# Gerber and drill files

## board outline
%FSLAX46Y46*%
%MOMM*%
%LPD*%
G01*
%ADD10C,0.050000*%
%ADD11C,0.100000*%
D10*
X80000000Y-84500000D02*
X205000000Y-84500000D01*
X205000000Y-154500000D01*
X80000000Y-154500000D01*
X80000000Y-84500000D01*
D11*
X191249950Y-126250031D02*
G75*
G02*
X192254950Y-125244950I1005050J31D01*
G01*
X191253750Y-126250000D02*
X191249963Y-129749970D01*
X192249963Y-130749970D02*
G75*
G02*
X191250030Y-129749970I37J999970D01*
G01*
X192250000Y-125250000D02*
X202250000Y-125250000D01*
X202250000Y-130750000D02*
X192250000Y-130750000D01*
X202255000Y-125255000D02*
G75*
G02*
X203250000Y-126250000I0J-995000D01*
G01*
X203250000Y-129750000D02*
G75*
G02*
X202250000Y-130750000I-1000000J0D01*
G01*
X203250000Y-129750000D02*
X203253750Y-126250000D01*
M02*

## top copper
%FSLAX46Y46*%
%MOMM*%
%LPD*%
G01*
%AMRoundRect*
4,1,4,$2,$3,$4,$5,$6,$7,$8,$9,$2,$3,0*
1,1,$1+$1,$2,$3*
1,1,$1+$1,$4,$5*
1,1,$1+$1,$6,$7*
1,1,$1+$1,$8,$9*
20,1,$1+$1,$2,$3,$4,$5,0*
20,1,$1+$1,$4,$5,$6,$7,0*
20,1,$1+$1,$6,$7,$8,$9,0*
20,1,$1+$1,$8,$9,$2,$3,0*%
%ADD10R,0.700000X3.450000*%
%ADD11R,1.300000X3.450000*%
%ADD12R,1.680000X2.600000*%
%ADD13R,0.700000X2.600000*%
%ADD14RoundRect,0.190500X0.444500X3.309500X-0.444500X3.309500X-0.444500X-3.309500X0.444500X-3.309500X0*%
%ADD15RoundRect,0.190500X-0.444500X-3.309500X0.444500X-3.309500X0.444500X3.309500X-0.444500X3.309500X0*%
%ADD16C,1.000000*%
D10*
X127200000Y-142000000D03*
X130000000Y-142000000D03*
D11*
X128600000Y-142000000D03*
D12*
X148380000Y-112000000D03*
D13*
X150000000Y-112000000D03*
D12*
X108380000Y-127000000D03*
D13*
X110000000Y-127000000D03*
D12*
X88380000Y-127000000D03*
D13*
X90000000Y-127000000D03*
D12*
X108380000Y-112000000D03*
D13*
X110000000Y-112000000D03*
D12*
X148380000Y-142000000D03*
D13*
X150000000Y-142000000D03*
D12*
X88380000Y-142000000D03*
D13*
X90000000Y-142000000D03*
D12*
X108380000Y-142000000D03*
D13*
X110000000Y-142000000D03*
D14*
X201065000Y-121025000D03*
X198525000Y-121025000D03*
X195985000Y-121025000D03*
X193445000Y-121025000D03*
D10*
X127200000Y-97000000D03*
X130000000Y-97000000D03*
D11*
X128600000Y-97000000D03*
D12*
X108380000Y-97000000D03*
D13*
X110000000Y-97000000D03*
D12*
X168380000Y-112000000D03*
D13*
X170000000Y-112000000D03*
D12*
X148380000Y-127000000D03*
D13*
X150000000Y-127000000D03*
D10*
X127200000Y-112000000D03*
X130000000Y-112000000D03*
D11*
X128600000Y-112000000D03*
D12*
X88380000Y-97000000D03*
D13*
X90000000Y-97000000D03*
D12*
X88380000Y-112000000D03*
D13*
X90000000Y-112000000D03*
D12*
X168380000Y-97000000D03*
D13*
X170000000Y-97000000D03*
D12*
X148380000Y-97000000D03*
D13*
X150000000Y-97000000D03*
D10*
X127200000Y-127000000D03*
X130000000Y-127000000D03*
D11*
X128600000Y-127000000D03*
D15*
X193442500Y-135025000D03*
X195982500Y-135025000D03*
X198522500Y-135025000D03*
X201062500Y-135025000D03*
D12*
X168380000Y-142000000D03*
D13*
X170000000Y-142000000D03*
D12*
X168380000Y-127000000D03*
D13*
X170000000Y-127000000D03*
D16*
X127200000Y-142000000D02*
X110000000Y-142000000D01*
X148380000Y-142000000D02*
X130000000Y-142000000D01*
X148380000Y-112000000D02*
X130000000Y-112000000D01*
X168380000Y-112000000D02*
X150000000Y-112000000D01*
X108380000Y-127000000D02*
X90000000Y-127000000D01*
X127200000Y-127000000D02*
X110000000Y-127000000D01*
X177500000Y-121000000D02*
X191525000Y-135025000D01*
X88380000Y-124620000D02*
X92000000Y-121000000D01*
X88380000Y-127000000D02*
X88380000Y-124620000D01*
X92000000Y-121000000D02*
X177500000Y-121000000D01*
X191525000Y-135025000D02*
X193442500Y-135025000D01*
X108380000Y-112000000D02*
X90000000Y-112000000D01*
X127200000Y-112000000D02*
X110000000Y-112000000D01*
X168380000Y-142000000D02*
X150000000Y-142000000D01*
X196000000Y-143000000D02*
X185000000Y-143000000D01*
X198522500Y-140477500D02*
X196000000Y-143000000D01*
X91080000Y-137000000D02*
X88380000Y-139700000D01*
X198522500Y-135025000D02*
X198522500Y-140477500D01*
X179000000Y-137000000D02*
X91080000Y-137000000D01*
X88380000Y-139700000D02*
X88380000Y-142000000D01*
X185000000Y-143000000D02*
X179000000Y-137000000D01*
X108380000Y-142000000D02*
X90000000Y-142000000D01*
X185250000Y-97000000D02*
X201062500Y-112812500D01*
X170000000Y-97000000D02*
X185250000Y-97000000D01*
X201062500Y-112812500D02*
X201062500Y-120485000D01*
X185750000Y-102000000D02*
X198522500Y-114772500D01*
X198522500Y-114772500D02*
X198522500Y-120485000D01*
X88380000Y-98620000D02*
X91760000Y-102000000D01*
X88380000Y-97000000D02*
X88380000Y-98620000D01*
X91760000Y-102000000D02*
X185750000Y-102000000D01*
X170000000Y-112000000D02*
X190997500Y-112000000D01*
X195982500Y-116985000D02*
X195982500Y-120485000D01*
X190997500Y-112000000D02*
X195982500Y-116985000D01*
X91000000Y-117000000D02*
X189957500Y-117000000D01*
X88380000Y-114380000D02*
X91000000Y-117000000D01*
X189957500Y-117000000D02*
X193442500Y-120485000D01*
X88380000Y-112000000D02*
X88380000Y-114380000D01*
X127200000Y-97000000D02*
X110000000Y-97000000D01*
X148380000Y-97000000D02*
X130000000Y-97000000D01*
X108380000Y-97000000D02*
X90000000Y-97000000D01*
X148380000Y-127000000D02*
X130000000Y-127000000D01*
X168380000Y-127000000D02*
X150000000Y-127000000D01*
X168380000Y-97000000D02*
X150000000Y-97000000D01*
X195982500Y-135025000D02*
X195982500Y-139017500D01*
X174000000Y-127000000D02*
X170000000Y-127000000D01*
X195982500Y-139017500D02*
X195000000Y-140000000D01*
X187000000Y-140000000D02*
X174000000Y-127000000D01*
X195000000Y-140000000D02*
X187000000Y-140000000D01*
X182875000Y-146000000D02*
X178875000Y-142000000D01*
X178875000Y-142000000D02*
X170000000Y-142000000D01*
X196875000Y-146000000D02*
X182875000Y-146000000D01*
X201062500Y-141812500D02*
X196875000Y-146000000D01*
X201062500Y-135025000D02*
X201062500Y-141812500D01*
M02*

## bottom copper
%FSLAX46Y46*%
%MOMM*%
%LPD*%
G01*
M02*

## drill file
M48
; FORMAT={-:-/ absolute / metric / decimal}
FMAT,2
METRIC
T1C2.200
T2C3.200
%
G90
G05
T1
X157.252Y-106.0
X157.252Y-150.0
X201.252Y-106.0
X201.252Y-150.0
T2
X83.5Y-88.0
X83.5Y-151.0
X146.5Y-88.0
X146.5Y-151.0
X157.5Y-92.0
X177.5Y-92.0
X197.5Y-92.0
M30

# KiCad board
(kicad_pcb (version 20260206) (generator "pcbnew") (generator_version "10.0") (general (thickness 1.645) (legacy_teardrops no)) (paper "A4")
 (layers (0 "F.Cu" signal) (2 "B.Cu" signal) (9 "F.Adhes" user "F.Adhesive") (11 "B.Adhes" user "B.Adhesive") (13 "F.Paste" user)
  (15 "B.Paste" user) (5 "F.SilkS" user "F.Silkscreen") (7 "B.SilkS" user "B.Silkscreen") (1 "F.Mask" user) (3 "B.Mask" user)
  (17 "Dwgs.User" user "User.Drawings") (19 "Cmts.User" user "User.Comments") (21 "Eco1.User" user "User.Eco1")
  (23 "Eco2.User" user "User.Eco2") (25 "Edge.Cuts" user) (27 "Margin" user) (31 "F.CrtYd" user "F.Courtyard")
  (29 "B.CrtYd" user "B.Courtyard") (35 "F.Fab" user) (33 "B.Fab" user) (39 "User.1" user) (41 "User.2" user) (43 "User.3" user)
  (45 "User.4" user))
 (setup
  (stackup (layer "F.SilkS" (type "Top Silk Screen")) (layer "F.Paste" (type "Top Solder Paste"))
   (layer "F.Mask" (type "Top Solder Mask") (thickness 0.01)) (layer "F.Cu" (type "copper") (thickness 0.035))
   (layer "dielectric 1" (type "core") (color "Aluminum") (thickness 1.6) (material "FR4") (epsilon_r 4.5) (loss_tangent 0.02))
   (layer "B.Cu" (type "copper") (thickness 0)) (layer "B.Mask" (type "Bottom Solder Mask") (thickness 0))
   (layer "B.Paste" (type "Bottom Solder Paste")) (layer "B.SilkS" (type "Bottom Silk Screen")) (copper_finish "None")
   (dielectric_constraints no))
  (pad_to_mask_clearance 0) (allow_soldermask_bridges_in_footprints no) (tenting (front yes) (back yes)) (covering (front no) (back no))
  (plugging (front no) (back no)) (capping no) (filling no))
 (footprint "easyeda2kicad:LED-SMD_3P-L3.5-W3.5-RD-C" (layer "F.Cu") (at 128.6 142)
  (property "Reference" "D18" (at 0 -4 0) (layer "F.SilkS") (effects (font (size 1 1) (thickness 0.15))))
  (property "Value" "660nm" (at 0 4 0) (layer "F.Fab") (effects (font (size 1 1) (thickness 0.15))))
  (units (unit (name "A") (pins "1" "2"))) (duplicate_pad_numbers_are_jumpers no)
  (pad "1" smd rect (at -1.4 0 180) (size 0.7 3.45) (layers "F.Cu" "F.Mask" "F.Paste") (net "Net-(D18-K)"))
  (pad "2" smd rect (at 1.4 0 180) (size 0.7 3.45) (layers "F.Cu" "F.Mask" "F.Paste") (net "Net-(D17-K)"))
  (pad "3" smd rect (at 0 0) (size 1.3 3.45) (layers "F.Cu" "F.Mask" "F.Paste")))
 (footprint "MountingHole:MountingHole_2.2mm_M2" (layer "F.Cu") (at 157.2525 106)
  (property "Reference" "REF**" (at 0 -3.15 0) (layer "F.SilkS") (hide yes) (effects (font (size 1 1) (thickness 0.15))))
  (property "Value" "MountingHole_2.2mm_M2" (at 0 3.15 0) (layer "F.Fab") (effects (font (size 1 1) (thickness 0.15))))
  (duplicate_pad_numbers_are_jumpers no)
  (pad "" np_thru_hole circle (at 0 0) (size 2.2 2.2) (drill 2.2) (layers "*.Cu" "*.Mask")))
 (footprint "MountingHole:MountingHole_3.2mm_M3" (layer "F.Cu") (at 83.5 88)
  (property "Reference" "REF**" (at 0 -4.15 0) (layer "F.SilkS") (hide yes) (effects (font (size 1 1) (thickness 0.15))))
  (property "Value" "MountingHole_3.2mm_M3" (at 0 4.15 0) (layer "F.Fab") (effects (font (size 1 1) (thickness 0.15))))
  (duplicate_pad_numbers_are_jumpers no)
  (pad "" np_thru_hole circle (at 0 0) (size 3.2 3.2) (drill 3.2) (layers "*.Cu" "*.Mask")))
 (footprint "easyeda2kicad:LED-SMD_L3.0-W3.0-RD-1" (layer "F.Cu") (at 149.19 112)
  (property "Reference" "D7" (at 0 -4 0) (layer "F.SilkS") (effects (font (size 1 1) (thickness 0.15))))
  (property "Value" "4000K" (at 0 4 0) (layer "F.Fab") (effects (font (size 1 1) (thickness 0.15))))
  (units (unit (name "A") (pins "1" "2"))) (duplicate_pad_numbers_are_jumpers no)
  (pad "1" smd rect (at -0.81 0 180) (size 1.68 2.6) (layers "F.Cu" "F.Mask" "F.Paste") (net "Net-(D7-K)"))
  (pad "2" smd rect (at 0.81 0 180) (size 0.7 2.6) (layers "F.Cu" "F.Mask" "F.Paste") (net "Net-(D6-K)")))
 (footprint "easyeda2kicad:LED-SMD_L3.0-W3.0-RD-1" (layer "F.Cu") (at 109.19 127)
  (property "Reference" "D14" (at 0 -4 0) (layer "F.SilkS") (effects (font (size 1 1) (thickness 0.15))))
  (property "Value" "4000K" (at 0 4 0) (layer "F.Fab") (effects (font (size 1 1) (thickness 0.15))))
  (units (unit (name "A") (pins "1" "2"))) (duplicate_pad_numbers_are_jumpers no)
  (pad "1" smd rect (at -0.81 0 180) (size 1.68 2.6) (layers "F.Cu" "F.Mask" "F.Paste") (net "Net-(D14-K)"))
  (pad "2" smd rect (at 0.81 0 180) (size 0.7 2.6) (layers "F.Cu" "F.Mask" "F.Paste") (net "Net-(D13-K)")))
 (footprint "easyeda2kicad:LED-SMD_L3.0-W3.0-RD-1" (layer "F.Cu") (at 89.19 127)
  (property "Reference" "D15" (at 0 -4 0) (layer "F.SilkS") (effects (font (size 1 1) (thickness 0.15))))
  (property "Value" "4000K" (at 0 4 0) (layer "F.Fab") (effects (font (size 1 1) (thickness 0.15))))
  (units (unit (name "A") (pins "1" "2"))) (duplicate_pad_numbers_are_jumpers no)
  (pad "1" smd rect (at -0.81 0 180) (size 1.68 2.6) (layers "F.Cu" "F.Mask" "F.Paste") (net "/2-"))
  (pad "2" smd rect (at 0.81 0 180) (size 0.7 2.6) (layers "F.Cu" "F.Mask" "F.Paste") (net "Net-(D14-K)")))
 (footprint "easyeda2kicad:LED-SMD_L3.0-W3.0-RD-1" (layer "F.Cu") (at 109.19 112)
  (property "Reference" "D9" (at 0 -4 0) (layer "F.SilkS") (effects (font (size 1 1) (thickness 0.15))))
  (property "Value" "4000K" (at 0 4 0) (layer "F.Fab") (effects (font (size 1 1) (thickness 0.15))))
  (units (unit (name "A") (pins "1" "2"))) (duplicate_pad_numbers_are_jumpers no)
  (pad "1" smd rect (at -0.81 0 180) (size 1.68 2.6) (layers "F.Cu" "F.Mask" "F.Paste") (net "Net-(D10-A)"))
  (pad "2" smd rect (at 0.81 0 180) (size 0.7 2.6) (layers "F.Cu" "F.Mask" "F.Paste") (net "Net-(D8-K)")))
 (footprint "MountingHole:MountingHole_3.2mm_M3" (layer "F.Cu") (at 83.5 151)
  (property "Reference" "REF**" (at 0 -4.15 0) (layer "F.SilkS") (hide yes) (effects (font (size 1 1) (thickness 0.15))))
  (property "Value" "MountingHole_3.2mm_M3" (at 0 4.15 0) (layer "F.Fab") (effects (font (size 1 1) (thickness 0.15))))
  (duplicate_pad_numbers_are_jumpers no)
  (pad "" np_thru_hole circle (at 0 0) (size 3.2 3.2) (drill 3.2) (layers "*.Cu" "*.Mask")))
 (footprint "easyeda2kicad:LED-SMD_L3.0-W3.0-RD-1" (layer "F.Cu") (at 149.19 142)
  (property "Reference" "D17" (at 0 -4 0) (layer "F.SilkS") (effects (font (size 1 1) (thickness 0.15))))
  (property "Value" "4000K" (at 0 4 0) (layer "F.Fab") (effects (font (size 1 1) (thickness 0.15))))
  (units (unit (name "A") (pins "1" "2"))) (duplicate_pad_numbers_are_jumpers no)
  (pad "1" smd rect (at -0.81 0 180) (size 1.68 2.6) (layers "F.Cu" "F.Mask" "F.Paste") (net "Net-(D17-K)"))
  (pad "2" smd rect (at 0.81 0 180) (size 0.7 2.6) (layers "F.Cu" "F.Mask" "F.Paste") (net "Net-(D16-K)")))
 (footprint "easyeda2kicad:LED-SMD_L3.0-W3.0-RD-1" (layer "F.Cu") (at 89.19 142)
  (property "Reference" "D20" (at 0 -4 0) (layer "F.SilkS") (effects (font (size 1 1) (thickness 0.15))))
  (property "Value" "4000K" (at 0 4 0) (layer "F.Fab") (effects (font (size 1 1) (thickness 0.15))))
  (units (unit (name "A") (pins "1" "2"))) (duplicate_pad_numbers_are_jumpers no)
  (pad "1" smd rect (at -0.81 0 180) (size 1.68 2.6) (layers "F.Cu" "F.Mask" "F.Paste") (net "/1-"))
  (pad "2" smd rect (at 0.81 0 180) (size 0.7 2.6) (layers "F.Cu" "F.Mask" "F.Paste") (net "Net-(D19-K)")))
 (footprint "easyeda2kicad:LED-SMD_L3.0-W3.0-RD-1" (layer "F.Cu") (at 109.19 142)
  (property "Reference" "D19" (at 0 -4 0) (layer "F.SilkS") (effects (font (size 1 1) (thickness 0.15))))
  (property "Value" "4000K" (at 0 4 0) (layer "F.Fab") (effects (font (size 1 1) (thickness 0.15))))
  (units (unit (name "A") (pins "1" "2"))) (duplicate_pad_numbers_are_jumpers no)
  (pad "1" smd rect (at -0.81 0 180) (size 1.68 2.6) (layers "F.Cu" "F.Mask" "F.Paste") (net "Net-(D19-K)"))
  (pad "2" smd rect (at 0.81 0 180) (size 0.7 2.6) (layers "F.Cu" "F.Mask" "F.Paste") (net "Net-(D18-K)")))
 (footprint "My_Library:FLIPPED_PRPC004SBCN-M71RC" (layer "F.Cu") (at 197.255 121.295 180)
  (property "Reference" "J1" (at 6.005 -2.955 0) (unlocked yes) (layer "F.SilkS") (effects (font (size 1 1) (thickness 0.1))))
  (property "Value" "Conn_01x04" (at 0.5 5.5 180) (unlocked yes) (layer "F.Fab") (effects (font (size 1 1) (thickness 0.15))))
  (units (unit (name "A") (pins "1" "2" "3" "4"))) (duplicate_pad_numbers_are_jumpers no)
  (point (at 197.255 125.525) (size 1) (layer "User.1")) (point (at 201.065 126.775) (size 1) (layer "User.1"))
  (pad "1" smd roundrect (at -3.81 0.27 180) (size 1.27 7) (layers "F.Cu" "F.Mask" "F.Paste") (roundrect_rratio 0.15) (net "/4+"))
  (pad "2" smd roundrect (at -1.27 0.27 180) (size 1.27 7) (layers "F.Cu" "F.Mask" "F.Paste") (roundrect_rratio 0.15) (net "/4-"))
  (pad "3" smd roundrect (at 1.27 0.27 180) (size 1.27 7) (layers "F.Cu" "F.Mask" "F.Paste") (roundrect_rratio 0.15) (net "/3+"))
  (pad "4" smd roundrect (at 3.81 0.27 180) (size 1.27 7) (layers "F.Cu" "F.Mask" "F.Paste") (roundrect_rratio 0.15) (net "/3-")))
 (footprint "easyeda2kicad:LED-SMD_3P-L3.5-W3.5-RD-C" (layer "F.Cu") (at 128.6 97)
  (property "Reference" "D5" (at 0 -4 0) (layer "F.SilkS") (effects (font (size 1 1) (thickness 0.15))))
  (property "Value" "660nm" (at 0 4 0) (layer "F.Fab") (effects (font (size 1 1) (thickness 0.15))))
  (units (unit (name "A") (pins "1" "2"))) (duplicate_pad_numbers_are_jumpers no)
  (pad "1" smd rect (at -1.4 0 180) (size 0.7 3.45) (layers "F.Cu" "F.Mask" "F.Paste") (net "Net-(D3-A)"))
  (pad "2" smd rect (at 1.4 0 180) (size 0.7 3.45) (layers "F.Cu" "F.Mask" "F.Paste") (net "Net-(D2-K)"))
  (pad "3" smd rect (at 0 0) (size 1.3 3.45) (layers "F.Cu" "F.Mask" "F.Paste")))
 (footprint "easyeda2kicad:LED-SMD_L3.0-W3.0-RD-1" (layer "F.Cu") (at 109.19 97)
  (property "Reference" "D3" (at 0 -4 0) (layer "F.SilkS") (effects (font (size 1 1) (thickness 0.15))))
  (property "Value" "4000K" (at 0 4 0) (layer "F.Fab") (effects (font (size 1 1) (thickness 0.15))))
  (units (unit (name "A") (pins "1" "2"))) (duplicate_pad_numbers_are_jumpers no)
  (pad "1" smd rect (at -0.81 0 180) (size 1.68 2.6) (layers "F.Cu" "F.Mask" "F.Paste") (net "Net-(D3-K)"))
  (pad "2" smd rect (at 0.81 0 180) (size 0.7 2.6) (layers "F.Cu" "F.Mask" "F.Paste") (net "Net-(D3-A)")))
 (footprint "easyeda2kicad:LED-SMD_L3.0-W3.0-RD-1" (layer "F.Cu") (at 169.19 112)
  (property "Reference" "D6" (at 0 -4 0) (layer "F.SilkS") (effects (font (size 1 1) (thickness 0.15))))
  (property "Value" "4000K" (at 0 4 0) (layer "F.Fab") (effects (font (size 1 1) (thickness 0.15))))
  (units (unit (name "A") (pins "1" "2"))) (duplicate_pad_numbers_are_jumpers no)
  (pad "1" smd rect (at -0.81 0 180) (size 1.68 2.6) (layers "F.Cu" "F.Mask" "F.Paste") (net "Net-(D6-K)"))
  (pad "2" smd rect (at 0.81 0 180) (size 0.7 2.6) (layers "F.Cu" "F.Mask" "F.Paste") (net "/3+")))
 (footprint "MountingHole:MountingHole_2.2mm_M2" (layer "F.Cu") (at 201.2525 106)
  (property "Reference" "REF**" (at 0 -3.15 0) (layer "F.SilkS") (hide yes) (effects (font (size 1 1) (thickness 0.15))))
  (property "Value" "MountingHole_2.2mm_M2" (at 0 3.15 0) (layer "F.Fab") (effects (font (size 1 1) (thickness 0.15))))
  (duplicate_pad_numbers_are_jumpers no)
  (pad "" np_thru_hole circle (at 0 0) (size 2.2 2.2) (drill 2.2) (layers "*.Cu" "*.Mask")))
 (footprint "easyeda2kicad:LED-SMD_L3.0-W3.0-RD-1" (layer "F.Cu") (at 149.19 127)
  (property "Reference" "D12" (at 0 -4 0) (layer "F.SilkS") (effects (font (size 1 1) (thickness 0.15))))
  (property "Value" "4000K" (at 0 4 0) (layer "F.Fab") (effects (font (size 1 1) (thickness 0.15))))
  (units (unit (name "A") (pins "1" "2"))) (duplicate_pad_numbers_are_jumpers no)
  (pad "1" smd rect (at -0.81 0 180) (size 1.68 2.6) (layers "F.Cu" "F.Mask" "F.Paste") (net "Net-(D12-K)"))
  (pad "2" smd rect (at 0.81 0 180) (size 0.7 2.6) (layers "F.Cu" "F.Mask" "F.Paste") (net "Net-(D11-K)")))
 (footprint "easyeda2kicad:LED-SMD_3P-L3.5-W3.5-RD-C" (layer "F.Cu") (at 128.6 112)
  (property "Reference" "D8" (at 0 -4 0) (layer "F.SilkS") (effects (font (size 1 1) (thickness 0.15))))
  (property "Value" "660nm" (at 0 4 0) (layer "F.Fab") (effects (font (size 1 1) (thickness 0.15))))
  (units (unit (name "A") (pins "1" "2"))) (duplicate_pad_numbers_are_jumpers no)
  (pad "1" smd rect (at -1.4 0 180) (size 0.7 3.45) (layers "F.Cu" "F.Mask" "F.Paste") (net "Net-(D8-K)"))
  (pad "2" smd rect (at 1.4 0 180) (size 0.7 3.45) (layers "F.Cu" "F.Mask" "F.Paste") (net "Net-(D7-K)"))
  (pad "3" smd rect (at 0 0) (size 1.3 3.45) (layers "F.Cu" "F.Mask" "F.Paste")))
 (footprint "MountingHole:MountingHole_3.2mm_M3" (layer "F.Cu") (at 146.5 151)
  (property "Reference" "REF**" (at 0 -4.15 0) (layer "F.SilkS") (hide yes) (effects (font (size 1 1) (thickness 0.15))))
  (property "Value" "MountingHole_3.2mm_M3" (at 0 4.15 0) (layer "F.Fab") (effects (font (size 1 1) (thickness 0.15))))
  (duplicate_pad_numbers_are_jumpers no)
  (pad "" np_thru_hole circle (at 0 0) (size 3.2 3.2) (drill 3.2) (layers "*.Cu" "*.Mask")))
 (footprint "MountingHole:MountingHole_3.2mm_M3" (layer "F.Cu") (at 177.5 92)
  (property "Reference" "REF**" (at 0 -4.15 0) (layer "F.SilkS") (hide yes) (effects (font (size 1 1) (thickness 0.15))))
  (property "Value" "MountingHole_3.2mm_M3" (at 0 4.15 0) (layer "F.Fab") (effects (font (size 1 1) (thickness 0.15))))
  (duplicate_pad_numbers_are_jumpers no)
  (pad "" np_thru_hole circle (at 0 0) (size 3.2 3.2) (drill 3.2) (layers "*.Cu" "*.Mask")))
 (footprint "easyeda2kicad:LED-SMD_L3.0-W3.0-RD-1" (layer "F.Cu") (at 89.19 97)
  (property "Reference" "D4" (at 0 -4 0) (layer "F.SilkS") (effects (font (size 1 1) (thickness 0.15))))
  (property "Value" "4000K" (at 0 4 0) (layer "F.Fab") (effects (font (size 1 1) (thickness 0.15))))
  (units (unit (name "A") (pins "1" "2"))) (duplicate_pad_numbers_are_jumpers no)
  (pad "1" smd rect (at -0.81 0 180) (size 1.68 2.6) (layers "F.Cu" "F.Mask" "F.Paste") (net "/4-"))
  (pad "2" smd rect (at 0.81 0 180) (size 0.7 2.6) (layers "F.Cu" "F.Mask" "F.Paste") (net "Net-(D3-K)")))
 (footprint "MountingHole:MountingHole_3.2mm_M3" (layer "F.Cu") (at 197.5 92)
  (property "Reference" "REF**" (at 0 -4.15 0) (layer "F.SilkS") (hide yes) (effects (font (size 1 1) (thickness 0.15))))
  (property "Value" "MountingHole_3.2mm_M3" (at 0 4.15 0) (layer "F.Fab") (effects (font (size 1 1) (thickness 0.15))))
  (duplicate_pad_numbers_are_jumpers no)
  (pad "" np_thru_hole circle (at 0 0) (size 3.2 3.2) (drill 3.2) (layers "*.Cu" "*.Mask")))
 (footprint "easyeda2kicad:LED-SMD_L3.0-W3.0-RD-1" (layer "F.Cu") (at 89.19 112)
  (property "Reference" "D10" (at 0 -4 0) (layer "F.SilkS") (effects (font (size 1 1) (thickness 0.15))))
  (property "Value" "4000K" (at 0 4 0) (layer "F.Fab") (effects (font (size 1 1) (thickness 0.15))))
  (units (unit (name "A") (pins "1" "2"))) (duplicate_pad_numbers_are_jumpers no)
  (pad "1" smd rect (at -0.81 0 180) (size 1.68 2.6) (layers "F.Cu" "F.Mask" "F.Paste") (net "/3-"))
  (pad "2" smd rect (at 0.81 0 180) (size 0.7 2.6) (layers "F.Cu" "F.Mask" "F.Paste") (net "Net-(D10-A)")))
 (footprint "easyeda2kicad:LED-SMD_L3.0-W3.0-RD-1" (layer "F.Cu") (at 169.19 97)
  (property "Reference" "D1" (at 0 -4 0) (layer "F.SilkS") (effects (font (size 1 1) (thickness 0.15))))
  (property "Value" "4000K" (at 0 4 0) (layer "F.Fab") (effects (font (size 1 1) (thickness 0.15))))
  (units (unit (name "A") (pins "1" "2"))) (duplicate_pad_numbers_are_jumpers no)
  (pad "1" smd rect (at -0.81 0 180) (size 1.68 2.6) (layers "F.Cu" "F.Mask" "F.Paste") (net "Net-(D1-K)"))
  (pad "2" smd rect (at 0.81 0 180) (size 0.7 2.6) (layers "F.Cu" "F.Mask" "F.Paste") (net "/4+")))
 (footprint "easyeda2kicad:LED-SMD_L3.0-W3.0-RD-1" (layer "F.Cu") (at 149.19 97)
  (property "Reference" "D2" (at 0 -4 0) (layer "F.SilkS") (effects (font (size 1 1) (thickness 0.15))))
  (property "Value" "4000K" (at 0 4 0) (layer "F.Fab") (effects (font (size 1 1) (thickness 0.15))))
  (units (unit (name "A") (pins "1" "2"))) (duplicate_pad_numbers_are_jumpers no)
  (pad "1" smd rect (at -0.81 0 180) (size 1.68 2.6) (layers "F.Cu" "F.Mask" "F.Paste") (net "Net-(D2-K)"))
  (pad "2" smd rect (at 0.81 0 180) (size 0.7 2.6) (layers "F.Cu" "F.Mask" "F.Paste") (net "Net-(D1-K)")))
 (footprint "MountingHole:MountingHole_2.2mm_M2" (layer "F.Cu") (at 157.2525 150)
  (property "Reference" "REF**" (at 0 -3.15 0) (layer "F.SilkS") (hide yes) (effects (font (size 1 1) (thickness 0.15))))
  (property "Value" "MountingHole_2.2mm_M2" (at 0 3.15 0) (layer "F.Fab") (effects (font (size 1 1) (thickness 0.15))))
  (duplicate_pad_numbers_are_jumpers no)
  (pad "" np_thru_hole circle (at 0 0) (size 2.2 2.2) (drill 2.2) (layers "*.Cu" "*.Mask")))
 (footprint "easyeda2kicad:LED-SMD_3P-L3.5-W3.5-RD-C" (layer "F.Cu") (at 128.6 127)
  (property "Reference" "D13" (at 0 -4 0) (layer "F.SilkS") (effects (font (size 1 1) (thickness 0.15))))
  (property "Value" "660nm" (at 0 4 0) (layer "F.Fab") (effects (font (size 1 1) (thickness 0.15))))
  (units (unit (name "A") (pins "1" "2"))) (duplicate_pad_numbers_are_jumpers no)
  (pad "1" smd rect (at -1.4 0 180) (size 0.7 3.45) (layers "F.Cu" "F.Mask" "F.Paste") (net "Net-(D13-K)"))
  (pad "2" smd rect (at 1.4 0 180) (size 0.7 3.45) (layers "F.Cu" "F.Mask" "F.Paste") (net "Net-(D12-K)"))
  (pad "3" smd rect (at 0 0) (size 1.3 3.45) (layers "F.Cu" "F.Mask" "F.Paste")))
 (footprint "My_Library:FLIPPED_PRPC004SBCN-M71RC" (layer "F.Cu") (at 197.2525 134.755)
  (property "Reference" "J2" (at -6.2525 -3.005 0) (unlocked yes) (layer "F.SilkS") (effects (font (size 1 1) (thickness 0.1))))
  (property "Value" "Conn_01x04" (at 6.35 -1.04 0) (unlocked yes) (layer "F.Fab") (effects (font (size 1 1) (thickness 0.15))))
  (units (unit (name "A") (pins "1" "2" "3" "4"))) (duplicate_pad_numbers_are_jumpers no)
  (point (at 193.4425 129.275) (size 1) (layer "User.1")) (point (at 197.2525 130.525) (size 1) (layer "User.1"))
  (pad "1" smd roundrect (at -3.81 0.27) (size 1.27 7) (layers "F.Cu" "F.Mask" "F.Paste") (roundrect_rratio 0.15) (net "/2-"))
  (pad "2" smd roundrect (at -1.27 0.27) (size 1.27 7) (layers "F.Cu" "F.Mask" "F.Paste") (roundrect_rratio 0.15) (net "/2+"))
  (pad "3" smd roundrect (at 1.27 0.27) (size 1.27 7) (layers "F.Cu" "F.Mask" "F.Paste") (roundrect_rratio 0.15) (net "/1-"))
  (pad "4" smd roundrect (at 3.81 0.27) (size 1.27 7) (layers "F.Cu" "F.Mask" "F.Paste") (roundrect_rratio 0.15) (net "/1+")))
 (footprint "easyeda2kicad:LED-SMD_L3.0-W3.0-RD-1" (layer "F.Cu") (at 169.19 142)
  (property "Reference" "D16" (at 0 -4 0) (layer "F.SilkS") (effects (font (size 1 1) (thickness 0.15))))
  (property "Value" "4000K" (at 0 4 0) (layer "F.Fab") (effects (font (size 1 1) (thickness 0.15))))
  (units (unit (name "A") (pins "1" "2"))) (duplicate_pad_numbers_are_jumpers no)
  (pad "1" smd rect (at -0.81 0 180) (size 1.68 2.6) (layers "F.Cu" "F.Mask" "F.Paste") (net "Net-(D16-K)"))
  (pad "2" smd rect (at 0.81 0 180) (size 0.7 2.6) (layers "F.Cu" "F.Mask" "F.Paste") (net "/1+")))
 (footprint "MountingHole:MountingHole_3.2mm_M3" (layer "F.Cu") (at 157.5 92)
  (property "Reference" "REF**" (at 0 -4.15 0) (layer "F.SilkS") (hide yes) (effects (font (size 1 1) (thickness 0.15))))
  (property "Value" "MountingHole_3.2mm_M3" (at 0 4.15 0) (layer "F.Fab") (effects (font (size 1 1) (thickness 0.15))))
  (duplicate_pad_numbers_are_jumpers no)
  (pad "" np_thru_hole circle (at 0 0) (size 3.2 3.2) (drill 3.2) (layers "*.Cu" "*.Mask")))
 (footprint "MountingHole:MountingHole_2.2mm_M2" (layer "F.Cu") (at 201.2525 150)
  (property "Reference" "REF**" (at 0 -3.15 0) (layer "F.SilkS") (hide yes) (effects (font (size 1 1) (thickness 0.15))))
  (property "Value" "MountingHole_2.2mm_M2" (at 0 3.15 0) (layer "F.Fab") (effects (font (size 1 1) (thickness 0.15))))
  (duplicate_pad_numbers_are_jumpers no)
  (pad "" np_thru_hole circle (at 0 0) (size 2.2 2.2) (drill 2.2) (layers "*.Cu" "*.Mask")))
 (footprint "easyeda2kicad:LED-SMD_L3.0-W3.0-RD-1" (layer "F.Cu") (at 169.19 127)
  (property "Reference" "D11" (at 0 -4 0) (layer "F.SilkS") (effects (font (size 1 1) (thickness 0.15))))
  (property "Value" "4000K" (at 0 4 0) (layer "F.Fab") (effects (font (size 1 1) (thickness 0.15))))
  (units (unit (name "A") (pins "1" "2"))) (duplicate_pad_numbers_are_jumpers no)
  (pad "1" smd rect (at -0.81 0 180) (size 1.68 2.6) (layers "F.Cu" "F.Mask" "F.Paste") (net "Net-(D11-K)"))
  (pad "2" smd rect (at 0.81 0 180) (size 0.7 2.6) (layers "F.Cu" "F.Mask" "F.Paste") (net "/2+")))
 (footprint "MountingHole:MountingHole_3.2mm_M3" (layer "F.Cu") (at 146.5 88)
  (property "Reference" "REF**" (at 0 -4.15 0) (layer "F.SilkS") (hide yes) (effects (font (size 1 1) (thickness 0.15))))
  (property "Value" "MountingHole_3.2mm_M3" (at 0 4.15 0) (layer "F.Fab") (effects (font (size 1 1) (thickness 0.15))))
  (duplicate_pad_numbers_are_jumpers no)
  (pad "" np_thru_hole circle (at 0 0) (size 3.2 3.2) (drill 3.2) (layers "*.Cu" "*.Mask")))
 (gr_rect (start 80 84.5) (end 205 154.5) (stroke (width 0.05) (type default)) (fill no) (layer "Edge.Cuts"))
 (gr_arc (start 191.24995 126.250031) (mid 191.544308 125.539389) (end 192.25495 125.245031) (stroke (width 0.1) (type default))
  (layer "Edge.Cuts"))
 (gr_line (start 191.25375 126.25) (end 191.249963 129.74997) (stroke (width 0.1) (type default)) (layer "Edge.Cuts"))
 (gr_arc (start 192.249963 130.74997) (mid 191.542857 130.457076) (end 191.249963 129.74997) (stroke (width 0.1) (type default))
  (layer "Edge.Cuts"))
 (gr_line (start 192.25 125.25) (end 202.25 125.25) (stroke (width 0.1) (type default)) (layer "Edge.Cuts"))
 (gr_line (start 202.25 130.75) (end 192.25 130.75) (stroke (width 0.1) (type default)) (layer "Edge.Cuts"))
 (gr_arc (start 202.255 125.255) (mid 202.958571 125.546429) (end 203.25 126.25) (stroke (width 0.1) (type default)) (layer "Edge.Cuts"))
 (gr_arc (start 203.25 129.75) (mid 202.957107 130.457107) (end 202.25 130.75) (stroke (width 0.1) (type default)) (layer "Edge.Cuts"))
 (gr_line (start 203.25 129.75) (end 203.25375 126.25) (stroke (width 0.1) (type default)) (layer "Edge.Cuts"))
 (segment (start 127.2 142) (end 110 142) (width 1) (layer "F.Cu") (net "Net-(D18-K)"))
 (segment (start 148.38 142) (end 130 142) (width 1) (layer "F.Cu") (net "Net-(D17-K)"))
 (segment (start 148.38 112) (end 130 112) (width 1) (layer "F.Cu") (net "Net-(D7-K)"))
 (segment (start 168.38 112) (end 150 112) (width 1) (layer "F.Cu") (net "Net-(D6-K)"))
 (segment (start 108.38 127) (end 90 127) (width 1) (layer "F.Cu") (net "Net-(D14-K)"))
 (segment (start 127.2 127) (end 110 127) (width 1) (layer "F.Cu") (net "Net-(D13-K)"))
 (segment (start 177.5 121) (end 191.525 135.025) (width 1) (layer "F.Cu") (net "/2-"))
 (segment (start 88.38 124.62) (end 92 121) (width 1) (layer "F.Cu") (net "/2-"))
 (segment (start 88.38 127) (end 88.38 124.62) (width 1) (layer "F.Cu") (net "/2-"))
 (segment (start 92 121) (end 177.5 121) (width 1) (layer "F.Cu") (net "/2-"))
 (segment (start 191.525 135.025) (end 193.4425 135.025) (width 1) (layer "F.Cu") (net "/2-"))
 (segment (start 108.38 112) (end 90 112) (width 1) (layer "F.Cu") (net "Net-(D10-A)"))
 (segment (start 127.2 112) (end 110 112) (width 1) (layer "F.Cu") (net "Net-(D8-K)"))
 (segment (start 168.38 142) (end 150 142) (width 1) (layer "F.Cu") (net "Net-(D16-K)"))
 (segment (start 196 143) (end 185 143) (width 1) (layer "F.Cu") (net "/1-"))
 (segment (start 198.5225 140.4775) (end 196 143) (width 1) (layer "F.Cu") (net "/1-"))
 (segment (start 91.08 137) (end 88.38 139.7) (width 1) (layer "F.Cu") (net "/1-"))
 (segment (start 198.5225 135.025) (end 198.5225 140.4775) (width 1) (layer "F.Cu") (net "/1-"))
 (segment (start 179 137) (end 91.08 137) (width 1) (layer "F.Cu") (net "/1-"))
 (segment (start 88.38 139.7) (end 88.38 142) (width 1) (layer "F.Cu") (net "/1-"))
 (segment (start 185 143) (end 179 137) (width 1) (layer "F.Cu") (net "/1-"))
 (segment (start 108.38 142) (end 90 142) (width 1) (layer "F.Cu") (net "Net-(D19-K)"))
 (segment (start 185.25 97) (end 201.0625 112.8125) (width 1) (layer "F.Cu") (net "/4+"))
 (segment (start 170 97) (end 185.25 97) (width 1) (layer "F.Cu") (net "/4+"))
 (segment (start 201.0625 112.8125) (end 201.0625 120.485) (width 1) (layer "F.Cu") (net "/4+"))
 (segment (start 185.75 102) (end 198.5225 114.7725) (width 1) (layer "F.Cu") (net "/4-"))
 (segment (start 198.5225 114.7725) (end 198.5225 120.485) (width 1) (layer "F.Cu") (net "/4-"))
 (segment (start 88.38 98.62) (end 91.76 102) (width 1) (layer "F.Cu") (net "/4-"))
 (segment (start 88.38 97) (end 88.38 98.62) (width 1) (layer "F.Cu") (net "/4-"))
 (segment (start 91.76 102) (end 185.75 102) (width 1) (layer "F.Cu") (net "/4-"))
 (segment (start 170 112) (end 190.9975 112) (width 1) (layer "F.Cu") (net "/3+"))
 (segment (start 195.9825 116.985) (end 195.9825 120.485) (width 1) (layer "F.Cu") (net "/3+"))
 (segment (start 190.9975 112) (end 195.9825 116.985) (width 1) (layer "F.Cu") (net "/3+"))
 (segment (start 91 117) (end 189.9575 117) (width 1) (layer "F.Cu") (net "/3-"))
 (segment (start 88.38 114.38) (end 91 117) (width 1) (layer "F.Cu") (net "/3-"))
 (segment (start 189.9575 117) (end 193.4425 120.485) (width 1) (layer "F.Cu") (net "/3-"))
 (segment (start 88.38 112) (end 88.38 114.38) (width 1) (layer "F.Cu") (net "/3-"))
 (segment (start 127.2 97) (end 110 97) (width 1) (layer "F.Cu") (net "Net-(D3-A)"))
 (segment (start 148.38 97) (end 130 97) (width 1) (layer "F.Cu") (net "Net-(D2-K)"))
 (segment (start 108.38 97) (end 90 97) (width 1) (layer "F.Cu") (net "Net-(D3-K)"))
 (segment (start 148.38 127) (end 130 127) (width 1) (layer "F.Cu") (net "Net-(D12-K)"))
 (segment (start 168.38 127) (end 150 127) (width 1) (layer "F.Cu") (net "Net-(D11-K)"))
 (segment (start 168.38 97) (end 150 97) (width 1) (layer "F.Cu") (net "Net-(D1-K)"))
 (segment (start 195.9825 135.025) (end 195.9825 139.0175) (width 1) (layer "F.Cu") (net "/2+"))
 (segment (start 174 127) (end 170 127) (width 1) (layer "F.Cu") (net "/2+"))
 (segment (start 195.9825 139.0175) (end 195 140) (width 1) (layer "F.Cu") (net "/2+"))
 (segment (start 187 140) (end 174 127) (width 1) (layer "F.Cu") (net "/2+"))
 (segment (start 195 140) (end 187 140) (width 1) (layer "F.Cu") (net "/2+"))
 (segment (start 182.875 146) (end 178.875 142) (width 1) (layer "F.Cu") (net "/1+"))
 (segment (start 178.875 142) (end 170 142) (width 1) (layer "F.Cu") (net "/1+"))
 (segment (start 196.875 146) (end 182.875 146) (width 1) (layer "F.Cu") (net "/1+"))
 (segment (start 201.0625 141.8125) (end 196.875 146) (width 1) (layer "F.Cu") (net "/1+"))
 (segment (start 201.0625 135.025) (end 201.0625 141.8125) (width 1) (layer "F.Cu") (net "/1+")))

